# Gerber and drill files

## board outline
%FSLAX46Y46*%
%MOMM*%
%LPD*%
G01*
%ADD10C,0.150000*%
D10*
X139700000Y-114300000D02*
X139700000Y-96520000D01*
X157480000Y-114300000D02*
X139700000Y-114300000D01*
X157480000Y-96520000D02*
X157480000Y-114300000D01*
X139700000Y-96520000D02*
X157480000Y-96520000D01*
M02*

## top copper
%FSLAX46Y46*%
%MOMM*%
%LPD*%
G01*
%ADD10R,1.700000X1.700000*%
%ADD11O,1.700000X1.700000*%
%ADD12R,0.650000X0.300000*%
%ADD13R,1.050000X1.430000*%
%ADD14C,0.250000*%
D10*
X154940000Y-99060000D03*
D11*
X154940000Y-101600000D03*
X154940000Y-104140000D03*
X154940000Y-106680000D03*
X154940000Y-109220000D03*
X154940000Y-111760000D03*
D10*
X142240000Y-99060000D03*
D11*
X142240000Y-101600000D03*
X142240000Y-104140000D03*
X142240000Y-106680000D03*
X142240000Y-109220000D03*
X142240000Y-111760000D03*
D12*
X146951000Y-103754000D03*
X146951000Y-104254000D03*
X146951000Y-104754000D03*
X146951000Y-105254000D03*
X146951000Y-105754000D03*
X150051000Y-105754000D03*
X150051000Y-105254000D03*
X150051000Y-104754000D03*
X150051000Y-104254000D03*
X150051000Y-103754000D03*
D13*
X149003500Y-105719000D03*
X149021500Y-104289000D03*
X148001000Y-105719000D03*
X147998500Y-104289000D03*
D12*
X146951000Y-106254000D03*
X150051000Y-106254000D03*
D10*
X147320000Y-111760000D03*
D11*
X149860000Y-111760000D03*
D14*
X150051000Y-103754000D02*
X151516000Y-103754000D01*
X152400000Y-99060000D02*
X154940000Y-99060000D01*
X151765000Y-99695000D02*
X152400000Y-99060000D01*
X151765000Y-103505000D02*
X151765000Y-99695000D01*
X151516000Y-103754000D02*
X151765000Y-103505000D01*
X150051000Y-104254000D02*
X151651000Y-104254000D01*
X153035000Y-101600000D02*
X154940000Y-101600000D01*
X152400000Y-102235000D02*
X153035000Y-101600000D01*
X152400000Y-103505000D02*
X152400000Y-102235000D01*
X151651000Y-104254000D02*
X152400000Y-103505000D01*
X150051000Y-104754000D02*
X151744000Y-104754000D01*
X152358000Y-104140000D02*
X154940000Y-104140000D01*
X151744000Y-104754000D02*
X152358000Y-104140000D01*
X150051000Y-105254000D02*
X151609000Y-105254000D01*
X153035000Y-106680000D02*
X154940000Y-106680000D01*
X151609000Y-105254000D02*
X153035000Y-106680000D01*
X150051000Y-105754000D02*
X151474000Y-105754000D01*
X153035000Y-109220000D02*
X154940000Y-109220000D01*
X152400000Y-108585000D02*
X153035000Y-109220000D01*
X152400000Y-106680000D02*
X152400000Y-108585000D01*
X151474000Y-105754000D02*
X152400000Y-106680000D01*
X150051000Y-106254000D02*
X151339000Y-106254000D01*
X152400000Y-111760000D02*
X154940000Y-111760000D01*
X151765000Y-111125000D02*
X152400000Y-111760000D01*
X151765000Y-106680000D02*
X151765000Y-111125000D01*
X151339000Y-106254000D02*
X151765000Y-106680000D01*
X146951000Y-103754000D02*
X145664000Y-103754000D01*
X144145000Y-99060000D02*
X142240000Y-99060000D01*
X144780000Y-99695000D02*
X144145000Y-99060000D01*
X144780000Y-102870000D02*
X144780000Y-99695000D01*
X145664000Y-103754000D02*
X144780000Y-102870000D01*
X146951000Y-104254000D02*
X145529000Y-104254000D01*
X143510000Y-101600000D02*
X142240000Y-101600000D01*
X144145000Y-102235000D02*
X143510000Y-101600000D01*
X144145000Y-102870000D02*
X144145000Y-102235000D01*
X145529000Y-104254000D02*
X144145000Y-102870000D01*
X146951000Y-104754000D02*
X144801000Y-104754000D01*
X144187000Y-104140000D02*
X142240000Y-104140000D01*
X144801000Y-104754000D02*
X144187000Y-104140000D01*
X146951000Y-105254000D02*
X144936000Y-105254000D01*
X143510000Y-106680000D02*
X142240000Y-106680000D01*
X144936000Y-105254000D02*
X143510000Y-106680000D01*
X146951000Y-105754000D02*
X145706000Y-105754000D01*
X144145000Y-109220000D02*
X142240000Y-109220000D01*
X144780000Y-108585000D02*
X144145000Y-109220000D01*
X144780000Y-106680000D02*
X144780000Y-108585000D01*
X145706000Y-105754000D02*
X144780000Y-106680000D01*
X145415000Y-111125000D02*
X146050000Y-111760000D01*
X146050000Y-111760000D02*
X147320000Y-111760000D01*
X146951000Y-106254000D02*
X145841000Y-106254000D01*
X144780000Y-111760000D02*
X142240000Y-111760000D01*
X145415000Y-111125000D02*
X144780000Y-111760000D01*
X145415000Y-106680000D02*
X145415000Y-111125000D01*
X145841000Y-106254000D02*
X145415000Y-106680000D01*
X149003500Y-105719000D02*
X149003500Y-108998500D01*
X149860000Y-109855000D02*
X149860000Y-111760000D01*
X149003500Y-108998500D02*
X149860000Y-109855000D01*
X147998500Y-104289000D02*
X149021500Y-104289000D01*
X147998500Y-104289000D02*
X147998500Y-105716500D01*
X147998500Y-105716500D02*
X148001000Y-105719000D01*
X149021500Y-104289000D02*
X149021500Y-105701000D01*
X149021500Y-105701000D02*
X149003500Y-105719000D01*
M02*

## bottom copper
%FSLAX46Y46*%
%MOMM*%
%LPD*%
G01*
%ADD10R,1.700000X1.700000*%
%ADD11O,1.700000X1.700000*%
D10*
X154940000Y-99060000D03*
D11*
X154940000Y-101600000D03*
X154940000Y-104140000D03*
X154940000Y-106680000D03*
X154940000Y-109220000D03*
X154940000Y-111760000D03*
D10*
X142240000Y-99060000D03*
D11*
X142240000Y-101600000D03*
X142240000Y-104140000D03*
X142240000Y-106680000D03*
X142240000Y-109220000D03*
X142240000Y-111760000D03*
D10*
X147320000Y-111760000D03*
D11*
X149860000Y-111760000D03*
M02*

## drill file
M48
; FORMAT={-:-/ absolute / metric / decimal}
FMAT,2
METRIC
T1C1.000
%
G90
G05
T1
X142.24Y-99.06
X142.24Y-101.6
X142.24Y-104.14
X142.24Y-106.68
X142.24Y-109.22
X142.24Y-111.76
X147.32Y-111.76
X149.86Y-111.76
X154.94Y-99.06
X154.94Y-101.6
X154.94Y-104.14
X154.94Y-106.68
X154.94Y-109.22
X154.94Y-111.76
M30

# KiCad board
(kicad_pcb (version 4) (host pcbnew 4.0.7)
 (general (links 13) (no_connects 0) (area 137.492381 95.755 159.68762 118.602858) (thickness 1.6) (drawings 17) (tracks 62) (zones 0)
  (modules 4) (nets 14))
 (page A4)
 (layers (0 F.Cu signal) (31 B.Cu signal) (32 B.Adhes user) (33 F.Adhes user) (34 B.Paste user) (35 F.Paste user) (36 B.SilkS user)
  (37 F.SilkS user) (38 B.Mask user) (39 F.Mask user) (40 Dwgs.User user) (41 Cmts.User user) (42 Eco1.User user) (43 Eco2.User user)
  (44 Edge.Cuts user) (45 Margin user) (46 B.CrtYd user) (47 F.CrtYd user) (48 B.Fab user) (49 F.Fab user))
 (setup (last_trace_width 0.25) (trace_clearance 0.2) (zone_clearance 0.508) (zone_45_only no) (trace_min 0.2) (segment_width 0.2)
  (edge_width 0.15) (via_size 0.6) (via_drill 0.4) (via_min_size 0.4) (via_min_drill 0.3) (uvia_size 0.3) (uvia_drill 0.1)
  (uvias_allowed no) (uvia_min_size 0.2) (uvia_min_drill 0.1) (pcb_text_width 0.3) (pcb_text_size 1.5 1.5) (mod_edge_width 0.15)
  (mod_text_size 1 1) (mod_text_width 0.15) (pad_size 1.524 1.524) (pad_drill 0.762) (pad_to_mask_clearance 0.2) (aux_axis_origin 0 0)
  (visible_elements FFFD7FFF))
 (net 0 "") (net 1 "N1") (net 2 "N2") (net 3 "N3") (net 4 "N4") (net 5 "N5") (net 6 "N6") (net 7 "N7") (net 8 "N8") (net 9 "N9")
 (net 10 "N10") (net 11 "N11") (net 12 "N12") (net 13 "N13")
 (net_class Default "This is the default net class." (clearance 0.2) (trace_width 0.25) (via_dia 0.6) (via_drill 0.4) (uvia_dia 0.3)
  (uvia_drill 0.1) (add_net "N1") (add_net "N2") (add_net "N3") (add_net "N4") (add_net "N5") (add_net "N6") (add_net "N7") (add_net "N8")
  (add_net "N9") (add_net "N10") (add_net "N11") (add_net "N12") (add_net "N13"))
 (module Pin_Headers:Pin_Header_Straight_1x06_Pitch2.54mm (layer F.Cu) (at 154.94 99.06)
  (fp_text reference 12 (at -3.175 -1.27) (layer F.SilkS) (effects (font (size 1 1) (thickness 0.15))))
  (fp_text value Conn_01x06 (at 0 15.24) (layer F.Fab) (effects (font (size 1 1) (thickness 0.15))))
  (pad 1 thru_hole rect (at 0 0) (size 1.7 1.7) (drill 1) (layers *.Cu *.Mask) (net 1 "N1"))
  (pad 2 thru_hole oval (at 0 2.54) (size 1.7 1.7) (drill 1) (layers *.Cu *.Mask) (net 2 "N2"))
  (pad 3 thru_hole oval (at 0 5.08) (size 1.7 1.7) (drill 1) (layers *.Cu *.Mask) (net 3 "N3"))
  (pad 4 thru_hole oval (at 0 7.62) (size 1.7 1.7) (drill 1) (layers *.Cu *.Mask) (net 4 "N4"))
  (pad 5 thru_hole oval (at 0 10.16) (size 1.7 1.7) (drill 1) (layers *.Cu *.Mask) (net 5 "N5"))
  (pad 6 thru_hole oval (at 0 12.7) (size 1.7 1.7) (drill 1) (layers *.Cu *.Mask) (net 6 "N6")))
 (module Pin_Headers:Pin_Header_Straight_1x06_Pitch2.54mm (layer F.Cu) (at 142.24 99.06)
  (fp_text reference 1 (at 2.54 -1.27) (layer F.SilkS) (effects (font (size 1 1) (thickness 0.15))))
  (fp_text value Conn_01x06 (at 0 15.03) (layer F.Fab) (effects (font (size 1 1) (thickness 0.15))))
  (pad 1 thru_hole rect (at 0 0) (size 1.7 1.7) (drill 1) (layers *.Cu *.Mask) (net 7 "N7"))
  (pad 2 thru_hole oval (at 0 2.54) (size 1.7 1.7) (drill 1) (layers *.Cu *.Mask) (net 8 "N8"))
  (pad 3 thru_hole oval (at 0 5.08) (size 1.7 1.7) (drill 1) (layers *.Cu *.Mask) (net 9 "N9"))
  (pad 4 thru_hole oval (at 0 7.62) (size 1.7 1.7) (drill 1) (layers *.Cu *.Mask) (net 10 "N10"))
  (pad 5 thru_hole oval (at 0 10.16) (size 1.7 1.7) (drill 1) (layers *.Cu *.Mask) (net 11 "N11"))
  (pad 6 thru_hole oval (at 0 12.7) (size 1.7 1.7) (drill 1) (layers *.Cu *.Mask) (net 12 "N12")))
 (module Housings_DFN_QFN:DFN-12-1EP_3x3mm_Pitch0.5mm (layer F.Cu) (at 148.501 105.004)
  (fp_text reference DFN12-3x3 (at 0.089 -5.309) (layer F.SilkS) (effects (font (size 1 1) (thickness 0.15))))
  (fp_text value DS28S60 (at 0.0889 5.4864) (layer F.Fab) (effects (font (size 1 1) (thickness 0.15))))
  (pad 1 smd rect (at -1.55 -1.25) (size 0.65 0.3) (layers F.Cu F.Paste F.Mask) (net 7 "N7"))
  (pad 2 smd rect (at -1.55 -0.75) (size 0.65 0.3) (layers F.Cu F.Paste F.Mask) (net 8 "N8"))
  (pad 3 smd rect (at -1.55 -0.25) (size 0.65 0.3) (layers F.Cu F.Paste F.Mask) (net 9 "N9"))
  (pad 4 smd rect (at -1.55 0.25) (size 0.65 0.3) (layers F.Cu F.Paste F.Mask) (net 10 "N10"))
  (pad 5 smd rect (at -1.55 0.75) (size 0.65 0.3) (layers F.Cu F.Paste F.Mask) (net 11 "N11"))
  (pad 8 smd rect (at 1.55 0.75) (size 0.65 0.3) (layers F.Cu F.Paste F.Mask))
  (pad 9 smd rect (at 1.55 0.25) (size 0.65 0.3) (layers F.Cu F.Paste F.Mask))
  (pad 10 smd rect (at 1.55 -0.25) (size 0.65 0.3) (layers F.Cu F.Paste F.Mask))
  (pad 11 smd rect (at 1.55 -0.75) (size 0.65 0.3) (layers F.Cu F.Paste F.Mask))
  (pad 12 smd rect (at 1.55 -1.25) (size 0.65 0.3) (layers F.Cu F.Paste F.Mask) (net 1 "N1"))
  (pad 13 smd rect (at 0.5025 0.715) (size 1.05 1.43) (layers F.Cu F.Paste F.Mask) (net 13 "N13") (solder_paste_margin_ratio -0.2))
  (pad 13 smd rect (at 0.5205 -0.715) (size 1.05 1.43) (layers F.Cu F.Paste F.Mask) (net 13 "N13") (solder_paste_margin_ratio -0.2))
  (pad 13 smd rect (at -0.5 0.715) (size 1.05 1.43) (layers F.Cu F.Paste F.Mask) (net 13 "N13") (solder_paste_margin_ratio -0.2))
  (pad 13 smd rect (at -0.5025 -0.715) (size 1.05 1.43) (layers F.Cu F.Paste F.Mask) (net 13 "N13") (solder_paste_margin_ratio -0.2))
  (pad 6 smd rect (at -1.55 1.25) (size 0.65 0.3) (layers F.Cu F.Paste F.Mask) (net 12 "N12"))
  (pad 7 smd rect (at 1.55 1.25) (size 0.65 0.3) (layers F.Cu F.Paste F.Mask) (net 6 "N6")))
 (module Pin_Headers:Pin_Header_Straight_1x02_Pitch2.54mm (layer F.Cu) (at 147.32 111.76 90)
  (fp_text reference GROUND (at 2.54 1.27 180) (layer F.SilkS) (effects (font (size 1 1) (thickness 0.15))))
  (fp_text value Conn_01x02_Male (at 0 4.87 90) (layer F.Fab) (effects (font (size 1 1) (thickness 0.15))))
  (pad 1 thru_hole rect (at 0 0 90) (size 1.7 1.7) (drill 1) (layers *.Cu *.Mask) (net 12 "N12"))
  (pad 2 thru_hole oval (at 0 2.54 90) (size 1.7 1.7) (drill 1) (layers *.Cu *.Mask) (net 13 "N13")))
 (gr_line (start 139.7 114.3) (end 139.7 96.52) (angle 90) (layer Edge.Cuts) (width 0.15))
 (gr_line (start 157.48 114.3) (end 139.7 114.3) (angle 90) (layer Edge.Cuts) (width 0.15))
 (gr_line (start 157.48 96.52) (end 157.48 114.3) (angle 90) (layer Edge.Cuts) (width 0.15))
 (gr_line (start 139.7 96.52) (end 157.48 96.52) (angle 90) (layer Edge.Cuts) (width 0.15))
 (segment (start 150.051 103.754) (end 151.516 103.754) (width 0.25) (layer F.Cu) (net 1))
 (segment (start 152.4 99.06) (end 154.94 99.06) (width 0.25) (layer F.Cu) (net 1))
 (segment (start 151.765 99.695) (end 152.4 99.06) (width 0.25) (layer F.Cu) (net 1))
 (segment (start 151.765 103.505) (end 151.765 99.695) (width 0.25) (layer F.Cu) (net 1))
 (segment (start 151.516 103.754) (end 151.765 103.505) (width 0.25) (layer F.Cu) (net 1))
 (segment (start 150.051 104.254) (end 151.651 104.254) (width 0.25) (layer F.Cu) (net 2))
 (segment (start 153.035 101.6) (end 154.94 101.6) (width 0.25) (layer F.Cu) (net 2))
 (segment (start 152.4 102.235) (end 153.035 101.6) (width 0.25) (layer F.Cu) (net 2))
 (segment (start 152.4 103.505) (end 152.4 102.235) (width 0.25) (layer F.Cu) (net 2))
 (segment (start 151.651 104.254) (end 152.4 103.505) (width 0.25) (layer F.Cu) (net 2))
 (segment (start 150.051 104.754) (end 151.744 104.754) (width 0.25) (layer F.Cu) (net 3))
 (segment (start 152.358 104.14) (end 154.94 104.14) (width 0.25) (layer F.Cu) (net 3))
 (segment (start 151.744 104.754) (end 152.358 104.14) (width 0.25) (layer F.Cu) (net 3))
 (segment (start 150.051 105.254) (end 151.609 105.254) (width 0.25) (layer F.Cu) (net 4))
 (segment (start 153.035 106.68) (end 154.94 106.68) (width 0.25) (layer F.Cu) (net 4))
 (segment (start 151.609 105.254) (end 153.035 106.68) (width 0.25) (layer F.Cu) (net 4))
 (segment (start 150.051 105.754) (end 151.474 105.754) (width 0.25) (layer F.Cu) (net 5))
 (segment (start 153.035 109.22) (end 154.94 109.22) (width 0.25) (layer F.Cu) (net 5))
 (segment (start 152.4 108.585) (end 153.035 109.22) (width 0.25) (layer F.Cu) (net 5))
 (segment (start 152.4 106.68) (end 152.4 108.585) (width 0.25) (layer F.Cu) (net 5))
 (segment (start 151.474 105.754) (end 152.4 106.68) (width 0.25) (layer F.Cu) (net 5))
 (segment (start 150.051 106.254) (end 151.339 106.254) (width 0.25) (layer F.Cu) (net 6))
 (segment (start 152.4 111.76) (end 154.94 111.76) (width 0.25) (layer F.Cu) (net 6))
 (segment (start 151.765 111.125) (end 152.4 111.76) (width 0.25) (layer F.Cu) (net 6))
 (segment (start 151.765 106.68) (end 151.765 111.125) (width 0.25) (layer F.Cu) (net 6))
 (segment (start 151.339 106.254) (end 151.765 106.68) (width 0.25) (layer F.Cu) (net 6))
 (segment (start 146.951 103.754) (end 145.664 103.754) (width 0.25) (layer F.Cu) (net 7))
 (segment (start 144.145 99.06) (end 142.24 99.06) (width 0.25) (layer F.Cu) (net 7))
 (segment (start 144.78 99.695) (end 144.145 99.06) (width 0.25) (layer F.Cu) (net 7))
 (segment (start 144.78 102.87) (end 144.78 99.695) (width 0.25) (layer F.Cu) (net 7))
 (segment (start 145.664 103.754) (end 144.78 102.87) (width 0.25) (layer F.Cu) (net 7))
 (segment (start 146.951 104.254) (end 145.529 104.254) (width 0.25) (layer F.Cu) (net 8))
 (segment (start 143.51 101.6) (end 142.24 101.6) (width 0.25) (layer F.Cu) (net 8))
 (segment (start 144.145 102.235) (end 143.51 101.6) (width 0.25) (layer F.Cu) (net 8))
 (segment (start 144.145 102.87) (end 144.145 102.235) (width 0.25) (layer F.Cu) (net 8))
 (segment (start 145.529 104.254) (end 144.145 102.87) (width 0.25) (layer F.Cu) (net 8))
 (segment (start 146.951 104.754) (end 144.801 104.754) (width 0.25) (layer F.Cu) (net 9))
 (segment (start 144.187 104.14) (end 142.24 104.14) (width 0.25) (layer F.Cu) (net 9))
 (segment (start 144.801 104.754) (end 144.187 104.14) (width 0.25) (layer F.Cu) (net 9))
 (segment (start 146.951 105.254) (end 144.936 105.254) (width 0.25) (layer F.Cu) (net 10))
 (segment (start 143.51 106.68) (end 142.24 106.68) (width 0.25) (layer F.Cu) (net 10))
 (segment (start 144.936 105.254) (end 143.51 106.68) (width 0.25) (layer F.Cu) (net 10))
 (segment (start 146.951 105.754) (end 145.706 105.754) (width 0.25) (layer F.Cu) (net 11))
 (segment (start 144.145 109.22) (end 142.24 109.22) (width 0.25) (layer F.Cu) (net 11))
 (segment (start 144.78 108.585) (end 144.145 109.22) (width 0.25) (layer F.Cu) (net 11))
 (segment (start 144.78 106.68) (end 144.78 108.585) (width 0.25) (layer F.Cu) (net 11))
 (segment (start 145.706 105.754) (end 144.78 106.68) (width 0.25) (layer F.Cu) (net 11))
 (segment (start 145.415 111.125) (end 146.05 111.76) (width 0.25) (layer F.Cu) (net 12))
 (segment (start 146.05 111.76) (end 147.32 111.76) (width 0.25) (layer F.Cu) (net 12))
 (segment (start 146.951 106.254) (end 145.841 106.254) (width 0.25) (layer F.Cu) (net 12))
 (segment (start 144.78 111.76) (end 142.24 111.76) (width 0.25) (layer F.Cu) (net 12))
 (segment (start 145.415 111.125) (end 144.78 111.76) (width 0.25) (layer F.Cu) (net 12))
 (segment (start 145.415 106.68) (end 145.415 111.125) (width 0.25) (layer F.Cu) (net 12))
 (segment (start 145.841 106.254) (end 145.415 106.68) (width 0.25) (layer F.Cu) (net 12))
 (segment (start 149.0035 105.719) (end 149.0035 108.9985) (width 0.25) (layer F.Cu) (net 13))
 (segment (start 149.86 109.855) (end 149.86 111.76) (width 0.25) (layer F.Cu) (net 13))
 (segment (start 149.0035 108.9985) (end 149.86 109.855) (width 0.25) (layer F.Cu) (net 13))
 (segment (start 147.9985 104.289) (end 149.0215 104.289) (width 0.25) (layer F.Cu) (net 13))
 (segment (start 147.9985 104.289) (end 147.9985 105.7165) (width 0.25) (layer F.Cu) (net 13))
 (segment (start 147.9985 105.7165) (end 148.001 105.719) (width 0.25) (layer F.Cu) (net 13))
 (segment (start 149.0215 104.289) (end 149.0215 105.701) (width 0.25) (layer F.Cu) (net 13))
 (segment (start 149.0215 105.701) (end 149.0035 105.719) (width 0.25) (layer F.Cu) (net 13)))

